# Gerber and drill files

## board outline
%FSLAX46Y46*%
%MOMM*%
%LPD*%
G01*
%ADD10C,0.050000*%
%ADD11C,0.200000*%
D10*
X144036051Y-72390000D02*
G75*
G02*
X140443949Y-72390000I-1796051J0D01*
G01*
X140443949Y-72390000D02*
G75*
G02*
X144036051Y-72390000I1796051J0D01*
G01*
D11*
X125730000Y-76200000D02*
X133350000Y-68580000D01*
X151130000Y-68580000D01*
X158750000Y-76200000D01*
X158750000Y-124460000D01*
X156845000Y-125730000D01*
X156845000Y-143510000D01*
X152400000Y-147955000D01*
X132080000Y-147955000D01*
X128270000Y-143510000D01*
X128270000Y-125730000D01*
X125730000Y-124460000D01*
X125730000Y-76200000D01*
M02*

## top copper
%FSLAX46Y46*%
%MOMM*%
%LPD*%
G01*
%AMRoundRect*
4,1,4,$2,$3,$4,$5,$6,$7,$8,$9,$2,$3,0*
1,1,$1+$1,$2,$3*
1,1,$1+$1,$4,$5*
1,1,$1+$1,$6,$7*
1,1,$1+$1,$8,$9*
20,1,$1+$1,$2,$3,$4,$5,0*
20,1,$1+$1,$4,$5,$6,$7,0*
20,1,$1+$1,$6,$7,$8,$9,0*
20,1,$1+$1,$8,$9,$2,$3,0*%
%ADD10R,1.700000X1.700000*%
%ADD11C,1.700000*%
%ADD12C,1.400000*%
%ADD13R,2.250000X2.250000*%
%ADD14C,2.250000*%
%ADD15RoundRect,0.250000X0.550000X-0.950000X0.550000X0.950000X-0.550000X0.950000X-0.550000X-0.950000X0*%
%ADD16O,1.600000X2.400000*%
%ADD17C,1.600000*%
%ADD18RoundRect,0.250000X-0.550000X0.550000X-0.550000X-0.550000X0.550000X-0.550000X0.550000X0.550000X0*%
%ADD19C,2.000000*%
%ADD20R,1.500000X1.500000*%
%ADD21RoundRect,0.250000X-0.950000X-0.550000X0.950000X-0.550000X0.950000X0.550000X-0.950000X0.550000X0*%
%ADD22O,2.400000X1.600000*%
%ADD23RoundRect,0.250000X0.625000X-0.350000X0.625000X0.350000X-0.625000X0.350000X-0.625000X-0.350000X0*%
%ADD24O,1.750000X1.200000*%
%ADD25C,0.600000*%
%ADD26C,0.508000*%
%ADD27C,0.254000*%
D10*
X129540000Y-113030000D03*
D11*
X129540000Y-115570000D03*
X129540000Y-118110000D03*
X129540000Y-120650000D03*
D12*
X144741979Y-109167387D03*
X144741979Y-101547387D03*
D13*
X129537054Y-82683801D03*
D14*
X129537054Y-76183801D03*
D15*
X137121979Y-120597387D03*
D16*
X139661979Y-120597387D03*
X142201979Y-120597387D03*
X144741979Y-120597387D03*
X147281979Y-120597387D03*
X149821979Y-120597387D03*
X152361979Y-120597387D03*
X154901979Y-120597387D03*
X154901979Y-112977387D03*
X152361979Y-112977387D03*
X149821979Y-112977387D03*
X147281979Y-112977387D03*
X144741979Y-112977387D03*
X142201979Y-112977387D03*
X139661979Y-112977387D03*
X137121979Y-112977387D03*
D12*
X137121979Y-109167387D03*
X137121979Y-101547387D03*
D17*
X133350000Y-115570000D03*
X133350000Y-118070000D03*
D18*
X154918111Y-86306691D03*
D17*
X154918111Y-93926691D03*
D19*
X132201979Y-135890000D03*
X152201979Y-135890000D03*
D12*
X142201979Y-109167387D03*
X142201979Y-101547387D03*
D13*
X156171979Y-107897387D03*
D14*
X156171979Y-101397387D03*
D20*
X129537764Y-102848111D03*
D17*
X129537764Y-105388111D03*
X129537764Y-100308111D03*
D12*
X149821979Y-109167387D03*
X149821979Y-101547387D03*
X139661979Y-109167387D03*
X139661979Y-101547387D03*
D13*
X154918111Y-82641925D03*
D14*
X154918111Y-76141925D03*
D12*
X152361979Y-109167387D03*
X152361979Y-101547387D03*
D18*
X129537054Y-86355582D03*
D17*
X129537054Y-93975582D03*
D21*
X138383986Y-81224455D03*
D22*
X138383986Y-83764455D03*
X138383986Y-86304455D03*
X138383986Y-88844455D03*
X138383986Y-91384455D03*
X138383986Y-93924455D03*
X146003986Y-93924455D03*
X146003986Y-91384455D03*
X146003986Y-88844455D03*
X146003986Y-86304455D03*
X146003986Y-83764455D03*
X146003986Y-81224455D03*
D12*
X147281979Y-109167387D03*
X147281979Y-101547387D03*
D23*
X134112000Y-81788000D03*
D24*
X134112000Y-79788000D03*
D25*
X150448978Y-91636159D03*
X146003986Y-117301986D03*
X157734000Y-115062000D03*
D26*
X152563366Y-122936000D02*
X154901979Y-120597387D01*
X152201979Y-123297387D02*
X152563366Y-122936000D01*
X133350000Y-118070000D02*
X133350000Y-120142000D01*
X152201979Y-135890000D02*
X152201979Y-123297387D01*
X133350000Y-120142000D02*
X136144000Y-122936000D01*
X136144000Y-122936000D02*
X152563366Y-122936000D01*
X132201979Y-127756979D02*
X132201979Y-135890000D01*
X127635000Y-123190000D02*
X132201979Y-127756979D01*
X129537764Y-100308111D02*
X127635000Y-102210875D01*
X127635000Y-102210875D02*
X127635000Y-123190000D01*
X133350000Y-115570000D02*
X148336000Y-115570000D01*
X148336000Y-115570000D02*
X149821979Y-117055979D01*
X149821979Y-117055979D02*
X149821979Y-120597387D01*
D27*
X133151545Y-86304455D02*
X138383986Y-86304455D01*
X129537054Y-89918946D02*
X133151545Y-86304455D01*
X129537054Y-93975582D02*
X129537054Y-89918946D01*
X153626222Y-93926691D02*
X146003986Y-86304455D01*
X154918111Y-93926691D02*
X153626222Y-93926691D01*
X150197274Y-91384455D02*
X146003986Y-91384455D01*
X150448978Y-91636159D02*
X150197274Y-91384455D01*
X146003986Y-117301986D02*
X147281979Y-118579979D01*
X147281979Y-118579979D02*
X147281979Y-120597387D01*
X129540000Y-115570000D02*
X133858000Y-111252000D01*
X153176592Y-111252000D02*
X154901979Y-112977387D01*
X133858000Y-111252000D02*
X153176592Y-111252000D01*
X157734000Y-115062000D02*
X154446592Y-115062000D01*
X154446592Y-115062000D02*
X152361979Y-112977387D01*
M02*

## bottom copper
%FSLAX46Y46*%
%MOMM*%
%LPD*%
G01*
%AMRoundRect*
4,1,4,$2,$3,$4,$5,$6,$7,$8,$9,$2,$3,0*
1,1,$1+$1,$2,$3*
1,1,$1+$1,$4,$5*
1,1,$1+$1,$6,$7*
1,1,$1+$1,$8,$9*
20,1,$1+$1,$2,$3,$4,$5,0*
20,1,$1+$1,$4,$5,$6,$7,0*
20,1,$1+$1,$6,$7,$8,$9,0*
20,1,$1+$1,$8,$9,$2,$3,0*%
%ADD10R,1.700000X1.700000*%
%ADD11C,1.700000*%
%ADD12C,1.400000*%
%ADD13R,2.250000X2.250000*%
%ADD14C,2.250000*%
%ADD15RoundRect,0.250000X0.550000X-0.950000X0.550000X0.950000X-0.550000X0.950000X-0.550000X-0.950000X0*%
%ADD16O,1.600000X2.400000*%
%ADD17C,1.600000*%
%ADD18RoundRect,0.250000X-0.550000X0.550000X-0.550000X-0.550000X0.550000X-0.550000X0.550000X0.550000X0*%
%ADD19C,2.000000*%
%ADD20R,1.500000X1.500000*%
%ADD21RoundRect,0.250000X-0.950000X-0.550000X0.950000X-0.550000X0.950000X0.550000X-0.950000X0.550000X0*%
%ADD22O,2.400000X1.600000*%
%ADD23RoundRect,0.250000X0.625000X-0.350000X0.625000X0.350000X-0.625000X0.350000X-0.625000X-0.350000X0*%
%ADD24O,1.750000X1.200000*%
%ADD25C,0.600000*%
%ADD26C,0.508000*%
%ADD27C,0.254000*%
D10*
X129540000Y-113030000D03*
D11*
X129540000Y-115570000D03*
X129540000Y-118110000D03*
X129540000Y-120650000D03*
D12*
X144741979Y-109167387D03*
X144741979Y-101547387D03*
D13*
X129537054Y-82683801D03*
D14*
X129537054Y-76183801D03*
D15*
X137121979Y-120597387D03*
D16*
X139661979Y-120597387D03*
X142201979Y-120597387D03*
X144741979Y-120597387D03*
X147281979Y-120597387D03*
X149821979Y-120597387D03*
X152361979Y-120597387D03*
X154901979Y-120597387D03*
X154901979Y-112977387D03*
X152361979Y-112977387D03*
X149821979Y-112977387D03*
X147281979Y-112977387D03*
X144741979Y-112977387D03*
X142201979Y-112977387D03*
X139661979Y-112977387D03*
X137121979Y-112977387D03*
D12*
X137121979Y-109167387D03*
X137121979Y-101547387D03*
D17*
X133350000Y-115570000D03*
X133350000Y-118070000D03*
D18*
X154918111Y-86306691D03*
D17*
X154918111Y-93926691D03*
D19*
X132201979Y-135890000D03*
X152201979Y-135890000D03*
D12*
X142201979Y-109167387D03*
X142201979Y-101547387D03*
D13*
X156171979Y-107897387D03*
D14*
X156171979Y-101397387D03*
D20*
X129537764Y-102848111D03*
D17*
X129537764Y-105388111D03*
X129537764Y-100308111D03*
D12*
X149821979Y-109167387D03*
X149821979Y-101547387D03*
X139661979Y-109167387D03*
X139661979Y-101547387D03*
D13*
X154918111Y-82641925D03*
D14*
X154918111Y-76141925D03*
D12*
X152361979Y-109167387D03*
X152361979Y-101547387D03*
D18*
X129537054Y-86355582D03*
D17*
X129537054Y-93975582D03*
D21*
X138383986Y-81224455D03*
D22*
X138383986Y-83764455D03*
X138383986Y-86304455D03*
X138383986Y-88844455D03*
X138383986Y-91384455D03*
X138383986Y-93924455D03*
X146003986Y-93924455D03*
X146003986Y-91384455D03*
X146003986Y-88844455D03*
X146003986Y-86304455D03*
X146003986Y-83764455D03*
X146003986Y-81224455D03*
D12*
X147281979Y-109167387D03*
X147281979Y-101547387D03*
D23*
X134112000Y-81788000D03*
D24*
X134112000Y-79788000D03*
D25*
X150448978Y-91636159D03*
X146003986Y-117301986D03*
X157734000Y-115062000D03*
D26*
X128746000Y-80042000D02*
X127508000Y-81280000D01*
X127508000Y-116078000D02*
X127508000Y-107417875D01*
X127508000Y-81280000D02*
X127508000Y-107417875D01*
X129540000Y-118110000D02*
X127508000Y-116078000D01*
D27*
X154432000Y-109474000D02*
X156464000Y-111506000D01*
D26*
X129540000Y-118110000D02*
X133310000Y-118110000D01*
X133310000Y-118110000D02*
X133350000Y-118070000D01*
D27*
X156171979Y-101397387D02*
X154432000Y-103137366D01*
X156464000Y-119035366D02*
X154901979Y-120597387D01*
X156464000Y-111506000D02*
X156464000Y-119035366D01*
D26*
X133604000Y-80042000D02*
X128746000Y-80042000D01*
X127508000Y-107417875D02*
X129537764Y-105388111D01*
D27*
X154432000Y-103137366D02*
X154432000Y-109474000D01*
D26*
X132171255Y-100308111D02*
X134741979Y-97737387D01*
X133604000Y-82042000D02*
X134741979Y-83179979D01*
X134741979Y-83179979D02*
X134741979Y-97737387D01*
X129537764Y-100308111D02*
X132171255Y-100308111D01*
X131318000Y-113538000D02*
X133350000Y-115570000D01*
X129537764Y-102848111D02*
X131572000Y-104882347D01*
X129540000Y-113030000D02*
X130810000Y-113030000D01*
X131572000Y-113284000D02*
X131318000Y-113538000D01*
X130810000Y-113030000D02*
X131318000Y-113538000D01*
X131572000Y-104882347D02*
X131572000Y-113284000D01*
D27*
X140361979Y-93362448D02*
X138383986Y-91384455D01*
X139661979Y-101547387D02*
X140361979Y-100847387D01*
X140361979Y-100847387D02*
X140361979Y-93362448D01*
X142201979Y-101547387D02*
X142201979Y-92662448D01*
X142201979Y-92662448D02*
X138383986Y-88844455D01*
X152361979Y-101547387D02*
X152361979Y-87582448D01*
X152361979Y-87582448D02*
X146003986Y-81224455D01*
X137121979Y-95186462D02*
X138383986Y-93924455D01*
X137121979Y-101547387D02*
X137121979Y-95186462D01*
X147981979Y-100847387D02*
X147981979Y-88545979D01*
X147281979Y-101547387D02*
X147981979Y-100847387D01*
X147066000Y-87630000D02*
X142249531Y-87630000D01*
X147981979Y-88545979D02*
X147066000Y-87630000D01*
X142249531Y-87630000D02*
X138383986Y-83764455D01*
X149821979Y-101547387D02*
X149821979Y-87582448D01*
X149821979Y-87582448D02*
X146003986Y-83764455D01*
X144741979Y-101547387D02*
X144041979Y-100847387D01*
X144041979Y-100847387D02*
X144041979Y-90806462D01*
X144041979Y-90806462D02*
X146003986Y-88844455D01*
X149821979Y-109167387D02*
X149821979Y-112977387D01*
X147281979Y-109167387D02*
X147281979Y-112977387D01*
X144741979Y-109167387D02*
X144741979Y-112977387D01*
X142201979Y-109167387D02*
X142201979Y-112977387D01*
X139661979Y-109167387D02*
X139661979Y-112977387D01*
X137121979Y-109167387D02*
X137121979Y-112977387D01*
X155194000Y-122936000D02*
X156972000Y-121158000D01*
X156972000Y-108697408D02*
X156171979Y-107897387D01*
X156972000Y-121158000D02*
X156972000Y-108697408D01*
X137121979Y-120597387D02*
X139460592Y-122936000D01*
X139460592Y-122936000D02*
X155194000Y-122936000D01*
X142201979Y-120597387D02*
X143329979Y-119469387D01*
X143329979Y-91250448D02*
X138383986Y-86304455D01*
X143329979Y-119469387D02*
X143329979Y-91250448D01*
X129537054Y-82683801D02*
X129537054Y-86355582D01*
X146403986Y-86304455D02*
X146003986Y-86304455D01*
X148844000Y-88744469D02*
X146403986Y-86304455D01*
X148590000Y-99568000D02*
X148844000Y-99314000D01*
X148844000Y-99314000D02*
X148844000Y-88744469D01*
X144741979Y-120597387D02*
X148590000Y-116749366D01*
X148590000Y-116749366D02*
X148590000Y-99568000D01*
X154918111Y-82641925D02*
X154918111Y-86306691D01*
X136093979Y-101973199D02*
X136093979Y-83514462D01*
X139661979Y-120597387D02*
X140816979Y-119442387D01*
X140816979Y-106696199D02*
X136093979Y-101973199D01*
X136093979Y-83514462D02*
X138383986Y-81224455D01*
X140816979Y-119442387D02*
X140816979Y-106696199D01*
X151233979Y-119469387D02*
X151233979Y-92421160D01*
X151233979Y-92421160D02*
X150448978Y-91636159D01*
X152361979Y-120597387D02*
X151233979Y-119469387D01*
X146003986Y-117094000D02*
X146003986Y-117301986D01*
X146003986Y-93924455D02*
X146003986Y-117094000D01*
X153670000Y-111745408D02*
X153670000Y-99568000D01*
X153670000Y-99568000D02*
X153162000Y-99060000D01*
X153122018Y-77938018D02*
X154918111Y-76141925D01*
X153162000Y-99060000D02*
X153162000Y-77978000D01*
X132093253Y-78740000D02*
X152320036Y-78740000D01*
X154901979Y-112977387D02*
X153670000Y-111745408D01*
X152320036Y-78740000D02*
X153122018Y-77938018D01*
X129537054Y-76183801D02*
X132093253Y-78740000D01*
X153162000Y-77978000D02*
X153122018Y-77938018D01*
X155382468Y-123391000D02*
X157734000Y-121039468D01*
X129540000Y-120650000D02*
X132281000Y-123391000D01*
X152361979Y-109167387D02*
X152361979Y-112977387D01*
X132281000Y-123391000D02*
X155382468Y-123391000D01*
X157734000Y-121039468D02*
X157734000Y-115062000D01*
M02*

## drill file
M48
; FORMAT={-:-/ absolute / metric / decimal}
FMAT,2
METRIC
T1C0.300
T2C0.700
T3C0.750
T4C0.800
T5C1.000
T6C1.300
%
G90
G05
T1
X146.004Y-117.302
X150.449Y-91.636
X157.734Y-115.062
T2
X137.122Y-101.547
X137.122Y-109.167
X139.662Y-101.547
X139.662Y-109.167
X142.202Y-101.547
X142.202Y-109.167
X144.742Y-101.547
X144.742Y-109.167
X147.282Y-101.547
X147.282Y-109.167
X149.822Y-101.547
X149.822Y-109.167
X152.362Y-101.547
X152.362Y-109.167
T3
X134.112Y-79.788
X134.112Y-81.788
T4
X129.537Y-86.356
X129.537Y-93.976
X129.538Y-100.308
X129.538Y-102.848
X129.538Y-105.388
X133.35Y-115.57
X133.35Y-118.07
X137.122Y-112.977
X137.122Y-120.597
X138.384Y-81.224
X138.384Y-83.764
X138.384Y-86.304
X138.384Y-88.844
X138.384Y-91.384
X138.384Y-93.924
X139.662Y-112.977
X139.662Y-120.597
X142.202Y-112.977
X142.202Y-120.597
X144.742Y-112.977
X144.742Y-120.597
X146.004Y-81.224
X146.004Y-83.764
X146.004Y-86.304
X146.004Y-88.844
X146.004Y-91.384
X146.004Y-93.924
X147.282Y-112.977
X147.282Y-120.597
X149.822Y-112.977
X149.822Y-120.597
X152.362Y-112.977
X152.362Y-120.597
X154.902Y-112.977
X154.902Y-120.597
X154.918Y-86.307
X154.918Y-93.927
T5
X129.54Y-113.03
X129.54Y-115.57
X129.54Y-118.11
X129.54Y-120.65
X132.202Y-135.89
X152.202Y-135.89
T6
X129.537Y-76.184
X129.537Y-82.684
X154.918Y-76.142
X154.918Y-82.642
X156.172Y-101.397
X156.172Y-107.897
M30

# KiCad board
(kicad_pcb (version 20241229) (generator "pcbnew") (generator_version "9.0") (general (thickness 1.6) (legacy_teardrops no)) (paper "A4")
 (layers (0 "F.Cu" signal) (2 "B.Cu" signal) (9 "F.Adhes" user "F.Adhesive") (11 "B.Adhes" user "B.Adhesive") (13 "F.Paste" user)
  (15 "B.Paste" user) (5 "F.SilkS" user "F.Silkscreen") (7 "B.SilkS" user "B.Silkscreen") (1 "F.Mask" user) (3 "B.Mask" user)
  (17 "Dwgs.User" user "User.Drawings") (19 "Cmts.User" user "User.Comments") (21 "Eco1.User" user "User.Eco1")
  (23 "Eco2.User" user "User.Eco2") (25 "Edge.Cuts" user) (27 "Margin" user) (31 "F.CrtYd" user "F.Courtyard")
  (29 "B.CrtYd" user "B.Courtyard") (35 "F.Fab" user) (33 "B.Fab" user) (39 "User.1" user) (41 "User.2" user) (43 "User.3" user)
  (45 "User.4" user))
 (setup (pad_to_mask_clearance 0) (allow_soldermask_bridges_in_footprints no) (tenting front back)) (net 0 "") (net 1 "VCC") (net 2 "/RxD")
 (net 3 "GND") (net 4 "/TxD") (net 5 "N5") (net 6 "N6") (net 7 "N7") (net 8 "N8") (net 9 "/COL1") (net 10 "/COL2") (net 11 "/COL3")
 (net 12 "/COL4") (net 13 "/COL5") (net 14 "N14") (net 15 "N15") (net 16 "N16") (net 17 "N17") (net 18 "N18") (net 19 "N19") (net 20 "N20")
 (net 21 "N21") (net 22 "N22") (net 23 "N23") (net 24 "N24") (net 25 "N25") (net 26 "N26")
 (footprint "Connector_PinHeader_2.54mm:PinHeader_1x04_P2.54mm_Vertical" (layer "F.Cu") (at 129.54 113.03)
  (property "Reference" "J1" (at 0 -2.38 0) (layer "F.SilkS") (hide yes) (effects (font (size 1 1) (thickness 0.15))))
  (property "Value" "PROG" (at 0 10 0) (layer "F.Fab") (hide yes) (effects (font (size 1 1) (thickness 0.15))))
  (pad "1" thru_hole rect (at 0 0) (size 1.7 1.7) (drill 1) (layers "*.Cu" "*.Mask") (remove_unused_layers no) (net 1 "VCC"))
  (pad "2" thru_hole circle (at 0 2.54) (size 1.7 1.7) (drill 1) (layers "*.Cu" "*.Mask") (remove_unused_layers no) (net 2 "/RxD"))
  (pad "3" thru_hole circle (at 0 5.08) (size 1.7 1.7) (drill 1) (layers "*.Cu" "*.Mask") (remove_unused_layers no) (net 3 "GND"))
  (pad "4" thru_hole circle (at 0 7.62) (size 1.7 1.7) (drill 1) (layers "*.Cu" "*.Mask") (remove_unused_layers no) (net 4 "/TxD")))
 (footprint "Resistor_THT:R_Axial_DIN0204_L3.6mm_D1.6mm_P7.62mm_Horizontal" (layer "F.Cu") (at 144.741979 109.167387 90)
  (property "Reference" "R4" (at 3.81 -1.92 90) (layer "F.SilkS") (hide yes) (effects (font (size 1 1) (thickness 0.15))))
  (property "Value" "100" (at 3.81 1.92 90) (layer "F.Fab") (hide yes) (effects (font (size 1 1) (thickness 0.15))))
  (pad "1" thru_hole circle (at 0 0 90) (size 1.4 1.4) (drill 0.7) (layers "*.Cu" "*.Mask") (remove_unused_layers no) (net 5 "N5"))
  (pad "2" thru_hole circle (at 7.62 0 90) (size 1.4 1.4) (drill 0.7) (layers "*.Cu" "*.Mask") (remove_unused_layers no) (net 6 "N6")))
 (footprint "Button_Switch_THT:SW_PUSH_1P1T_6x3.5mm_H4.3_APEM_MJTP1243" (layer "F.Cu") (at 129.537054 82.683801 90)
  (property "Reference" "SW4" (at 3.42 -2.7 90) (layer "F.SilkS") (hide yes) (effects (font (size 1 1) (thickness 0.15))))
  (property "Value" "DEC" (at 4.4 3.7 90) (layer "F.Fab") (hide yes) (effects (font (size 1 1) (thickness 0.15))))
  (pad "1" thru_hole rect (at 0 0 180) (size 2.25 2.25) (drill 1.3) (layers "*.Cu" "*.Mask") (remove_unused_layers no) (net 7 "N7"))
  (pad "2" thru_hole circle (at 6.5 0 180) (size 2.25 2.25) (drill 1.3) (layers "*.Cu" "*.Mask") (remove_unused_layers no) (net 2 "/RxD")))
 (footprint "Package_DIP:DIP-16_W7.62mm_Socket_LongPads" (layer "F.Cu") (at 137.121979 120.597387 90)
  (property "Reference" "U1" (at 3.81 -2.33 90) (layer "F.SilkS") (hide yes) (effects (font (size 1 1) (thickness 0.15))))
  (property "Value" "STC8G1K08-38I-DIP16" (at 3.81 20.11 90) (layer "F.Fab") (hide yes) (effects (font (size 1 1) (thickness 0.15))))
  (pad "1" thru_hole roundrect (at 0 0 90) (size 2.4 1.6) (drill 0.8) (layers "*.Cu" "*.Mask") (remove_unused_layers no)
   (roundrect_rratio 0.15625) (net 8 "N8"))
  (pad "2" thru_hole oval (at 0 2.54 90) (size 2.4 1.6) (drill 0.8) (layers "*.Cu" "*.Mask") (remove_unused_layers no) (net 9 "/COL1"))
  (pad "3" thru_hole oval (at 0 5.08 90) (size 2.4 1.6) (drill 0.8) (layers "*.Cu" "*.Mask") (remove_unused_layers no) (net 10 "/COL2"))
  (pad "4" thru_hole oval (at 0 7.62 90) (size 2.4 1.6) (drill 0.8) (layers "*.Cu" "*.Mask") (remove_unused_layers no) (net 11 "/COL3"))
  (pad "5" thru_hole oval (at 0 10.16 90) (size 2.4 1.6) (drill 0.8) (layers "*.Cu" "*.Mask") (remove_unused_layers no) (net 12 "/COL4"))
  (pad "6" thru_hole oval (at 0 12.7 90) (size 2.4 1.6) (drill 0.8) (layers "*.Cu" "*.Mask") (remove_unused_layers no) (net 1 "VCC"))
  (pad "7" thru_hole oval (at 0 15.24 90) (size 2.4 1.6) (drill 0.8) (layers "*.Cu" "*.Mask") (remove_unused_layers no) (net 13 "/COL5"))
  (pad "8" thru_hole oval (at 0 17.78 90) (size 2.4 1.6) (drill 0.8) (layers "*.Cu" "*.Mask") (remove_unused_layers no) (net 3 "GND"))
  (pad "9" thru_hole oval (at 7.62 17.78 90) (size 2.4 1.6) (drill 0.8) (layers "*.Cu" "*.Mask") (remove_unused_layers no) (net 2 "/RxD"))
  (pad "10" thru_hole oval (at 7.62 15.24 90) (size 2.4 1.6) (drill 0.8) (layers "*.Cu" "*.Mask") (remove_unused_layers no) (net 4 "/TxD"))
  (pad "11" thru_hole oval (at 7.62 12.7 90) (size 2.4 1.6) (drill 0.8) (layers "*.Cu" "*.Mask") (remove_unused_layers no) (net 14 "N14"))
  (pad "12" thru_hole oval (at 7.62 10.16 90) (size 2.4 1.6) (drill 0.8) (layers "*.Cu" "*.Mask") (remove_unused_layers no) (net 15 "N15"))
  (pad "13" thru_hole oval (at 7.62 7.62 90) (size 2.4 1.6) (drill 0.8) (layers "*.Cu" "*.Mask") (remove_unused_layers no) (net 5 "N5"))
  (pad "14" thru_hole oval (at 7.62 5.08 90) (size 2.4 1.6) (drill 0.8) (layers "*.Cu" "*.Mask") (remove_unused_layers no) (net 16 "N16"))
  (pad "15" thru_hole oval (at 7.62 2.54 90) (size 2.4 1.6) (drill 0.8) (layers "*.Cu" "*.Mask") (remove_unused_layers no) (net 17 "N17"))
  (pad "16" thru_hole oval (at 7.62 0 90) (size 2.4 1.6) (drill 0.8) (layers "*.Cu" "*.Mask") (remove_unused_layers no) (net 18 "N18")))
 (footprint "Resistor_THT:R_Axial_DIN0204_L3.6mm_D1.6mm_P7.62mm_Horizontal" (layer "F.Cu") (at 137.121979 109.167387 90)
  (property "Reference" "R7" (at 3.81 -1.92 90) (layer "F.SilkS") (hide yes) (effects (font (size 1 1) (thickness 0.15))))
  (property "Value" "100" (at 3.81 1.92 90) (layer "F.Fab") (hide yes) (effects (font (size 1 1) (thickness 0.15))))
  (pad "1" thru_hole circle (at 0 0 90) (size 1.4 1.4) (drill 0.7) (layers "*.Cu" "*.Mask") (remove_unused_layers no) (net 18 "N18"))
  (pad "2" thru_hole circle (at 7.62 0 90) (size 1.4 1.4) (drill 0.7) (layers "*.Cu" "*.Mask") (remove_unused_layers no) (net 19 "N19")))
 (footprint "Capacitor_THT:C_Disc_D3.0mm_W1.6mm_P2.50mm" (layer "F.Cu") (at 133.35 115.57 -90)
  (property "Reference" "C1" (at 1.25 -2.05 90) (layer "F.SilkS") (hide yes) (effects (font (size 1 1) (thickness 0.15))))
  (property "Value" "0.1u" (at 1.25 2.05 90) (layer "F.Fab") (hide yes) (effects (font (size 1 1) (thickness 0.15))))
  (pad "1" thru_hole circle (at 0 0 270) (size 1.6 1.6) (drill 0.8) (layers "*.Cu" "*.Mask") (remove_unused_layers no) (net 1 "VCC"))
  (pad "2" thru_hole circle (at 2.5 0 270) (size 1.6 1.6) (drill 0.8) (layers "*.Cu" "*.Mask") (remove_unused_layers no) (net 3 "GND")))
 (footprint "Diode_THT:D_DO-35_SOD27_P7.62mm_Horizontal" (layer "F.Cu") (at 154.918111 86.306691 -90)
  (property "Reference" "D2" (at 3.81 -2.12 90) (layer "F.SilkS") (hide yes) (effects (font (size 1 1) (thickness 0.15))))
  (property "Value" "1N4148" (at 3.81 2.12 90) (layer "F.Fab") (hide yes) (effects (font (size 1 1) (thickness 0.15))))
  (pad "1" thru_hole roundrect (at 0 0 270) (size 1.6 1.6) (drill 0.8) (layers "*.Cu" "*.Mask") (remove_unused_layers no)
   (roundrect_rratio 0.15625) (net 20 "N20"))
  (pad "2" thru_hole circle (at 7.62 0 270) (size 1.6 1.6) (drill 0.8) (layers "*.Cu" "*.Mask") (remove_unused_layers no) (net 11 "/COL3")))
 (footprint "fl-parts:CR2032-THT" (layer "F.Cu") (at 142.201979 135.89 180)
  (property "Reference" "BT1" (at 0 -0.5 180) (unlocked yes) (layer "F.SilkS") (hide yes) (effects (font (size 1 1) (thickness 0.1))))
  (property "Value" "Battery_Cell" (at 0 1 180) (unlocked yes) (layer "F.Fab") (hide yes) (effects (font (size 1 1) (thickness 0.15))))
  (pad "1" thru_hole circle (at 10 0 180) (size 2 2) (drill 1) (layers "*.Cu" "*.Mask") (remove_unused_layers no) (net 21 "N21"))
  (pad "2" thru_hole circle (at -10 0 180) (size 2 2) (drill 1) (layers "*.Cu" "*.Mask") (remove_unused_layers no) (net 3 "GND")))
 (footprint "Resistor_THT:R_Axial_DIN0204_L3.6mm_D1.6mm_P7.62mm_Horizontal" (layer "F.Cu") (at 142.201979 109.167387 90)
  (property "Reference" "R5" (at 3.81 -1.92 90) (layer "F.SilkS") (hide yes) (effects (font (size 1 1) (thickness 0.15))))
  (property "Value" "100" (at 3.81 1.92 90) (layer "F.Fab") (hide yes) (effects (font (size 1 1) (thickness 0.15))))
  (pad "1" thru_hole circle (at 0 0 90) (size 1.4 1.4) (drill 0.7) (layers "*.Cu" "*.Mask") (remove_unused_layers no) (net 16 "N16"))
  (pad "2" thru_hole circle (at 7.62 0 90) (size 1.4 1.4) (drill 0.7) (layers "*.Cu" "*.Mask") (remove_unused_layers no) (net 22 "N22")))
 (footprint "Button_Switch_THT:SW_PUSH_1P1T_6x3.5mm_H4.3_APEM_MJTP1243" (layer "F.Cu") (at 156.171979 107.897387 90)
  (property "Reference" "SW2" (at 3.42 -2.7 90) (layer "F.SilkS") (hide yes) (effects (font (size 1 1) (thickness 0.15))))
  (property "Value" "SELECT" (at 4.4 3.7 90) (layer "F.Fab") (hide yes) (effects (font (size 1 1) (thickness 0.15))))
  (pad "1" thru_hole rect (at 0 0 180) (size 2.25 2.25) (drill 1.3) (layers "*.Cu" "*.Mask") (remove_unused_layers no) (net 8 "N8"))
  (pad "2" thru_hole circle (at 6.5 0 180) (size 2.25 2.25) (drill 1.3) (layers "*.Cu" "*.Mask") (remove_unused_layers no) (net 3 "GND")))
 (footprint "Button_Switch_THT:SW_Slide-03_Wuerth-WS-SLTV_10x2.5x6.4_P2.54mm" (layer "F.Cu") (at 129.537764 102.848111 90)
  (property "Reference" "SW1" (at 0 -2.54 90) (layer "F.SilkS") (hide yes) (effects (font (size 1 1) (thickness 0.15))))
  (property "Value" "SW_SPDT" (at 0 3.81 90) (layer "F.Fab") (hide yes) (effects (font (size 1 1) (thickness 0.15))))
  (pad "1" thru_hole rect (at 0 0 90) (size 1.5 1.5) (drill 0.8) (layers "*.Cu" "*.Mask") (remove_unused_layers no) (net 1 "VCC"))
  (pad "2" thru_hole circle (at -2.54 0 90) (size 1.6 1.6) (drill 0.8) (layers "*.Cu" "*.Mask") (remove_unused_layers no) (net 3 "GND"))
  (pad "3" thru_hole circle (at 2.54 0 90) (size 1.6 1.6) (drill 0.8) (layers "*.Cu" "*.Mask") (remove_unused_layers no) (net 21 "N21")))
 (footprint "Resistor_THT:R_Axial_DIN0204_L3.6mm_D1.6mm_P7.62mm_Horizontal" (layer "F.Cu") (at 149.821979 109.167387 90)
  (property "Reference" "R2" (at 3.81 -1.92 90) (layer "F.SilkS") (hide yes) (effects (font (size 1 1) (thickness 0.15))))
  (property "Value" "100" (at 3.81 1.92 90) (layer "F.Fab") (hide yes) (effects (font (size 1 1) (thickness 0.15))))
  (pad "1" thru_hole circle (at 0 0 90) (size 1.4 1.4) (drill 0.7) (layers "*.Cu" "*.Mask") (remove_unused_layers no) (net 14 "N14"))
  (pad "2" thru_hole circle (at 7.62 0 90) (size 1.4 1.4) (drill 0.7) (layers "*.Cu" "*.Mask") (remove_unused_layers no) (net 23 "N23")))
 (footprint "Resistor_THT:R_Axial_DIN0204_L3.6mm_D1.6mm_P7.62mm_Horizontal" (layer "F.Cu") (at 139.661979 109.167387 90)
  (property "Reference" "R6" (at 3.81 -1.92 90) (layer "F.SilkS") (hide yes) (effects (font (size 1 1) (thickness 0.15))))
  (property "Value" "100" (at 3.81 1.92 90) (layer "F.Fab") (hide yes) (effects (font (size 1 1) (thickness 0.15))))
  (pad "1" thru_hole circle (at 0 0 90) (size 1.4 1.4) (drill 0.7) (layers "*.Cu" "*.Mask") (remove_unused_layers no) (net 17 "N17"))
  (pad "2" thru_hole circle (at 7.62 0 90) (size 1.4 1.4) (drill 0.7) (layers "*.Cu" "*.Mask") (remove_unused_layers no) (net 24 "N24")))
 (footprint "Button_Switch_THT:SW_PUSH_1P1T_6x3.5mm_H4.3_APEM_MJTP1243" (layer "F.Cu") (at 154.918111 82.641925 90)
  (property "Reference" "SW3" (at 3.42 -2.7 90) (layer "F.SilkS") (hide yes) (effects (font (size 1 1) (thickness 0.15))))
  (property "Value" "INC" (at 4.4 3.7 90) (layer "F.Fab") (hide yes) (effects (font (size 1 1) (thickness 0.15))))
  (pad "1" thru_hole rect (at 0 0 180) (size 2.25 2.25) (drill 1.3) (layers "*.Cu" "*.Mask") (remove_unused_layers no) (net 20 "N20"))
  (pad "2" thru_hole circle (at 6.5 0 180) (size 2.25 2.25) (drill 1.3) (layers "*.Cu" "*.Mask") (remove_unused_layers no) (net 2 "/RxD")))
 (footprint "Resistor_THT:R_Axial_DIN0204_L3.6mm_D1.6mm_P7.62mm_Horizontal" (layer "F.Cu") (at 152.361979 109.167387 90)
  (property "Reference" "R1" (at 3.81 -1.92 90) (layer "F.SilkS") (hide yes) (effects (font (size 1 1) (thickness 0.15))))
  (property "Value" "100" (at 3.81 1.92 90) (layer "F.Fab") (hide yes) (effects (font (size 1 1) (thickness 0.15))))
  (pad "1" thru_hole circle (at 0 0 90) (size 1.4 1.4) (drill 0.7) (layers "*.Cu" "*.Mask") (remove_unused_layers no) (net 4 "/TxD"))
  (pad "2" thru_hole circle (at 7.62 0 90) (size 1.4 1.4) (drill 0.7) (layers "*.Cu" "*.Mask") (remove_unused_layers no) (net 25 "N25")))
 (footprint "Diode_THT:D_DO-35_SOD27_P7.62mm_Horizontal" (layer "F.Cu") (at 129.537054 86.355582 -90)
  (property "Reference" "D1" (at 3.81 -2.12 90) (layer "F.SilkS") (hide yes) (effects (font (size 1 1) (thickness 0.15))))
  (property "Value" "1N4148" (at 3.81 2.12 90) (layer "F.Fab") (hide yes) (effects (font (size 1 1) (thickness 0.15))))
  (pad "1" thru_hole roundrect (at 0 0 270) (size 1.6 1.6) (drill 0.8) (layers "*.Cu" "*.Mask") (remove_unused_layers no)
   (roundrect_rratio 0.15625) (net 7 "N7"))
  (pad "2" thru_hole circle (at 7.62 0 270) (size 1.6 1.6) (drill 0.8) (layers "*.Cu" "*.Mask") (remove_unused_layers no) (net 10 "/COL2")))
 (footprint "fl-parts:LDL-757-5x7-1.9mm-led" (layer "F.Cu") (at 138.383986 81.224455)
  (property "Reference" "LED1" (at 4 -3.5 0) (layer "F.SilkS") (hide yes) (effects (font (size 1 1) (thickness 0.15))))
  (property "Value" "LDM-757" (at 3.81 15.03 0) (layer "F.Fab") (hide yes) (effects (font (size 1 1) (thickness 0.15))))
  (pad "1" thru_hole roundrect (at 0 0) (size 2.4 1.6) (drill 0.8) (layers "*.Cu" "*.Mask") (remove_unused_layers no)
   (roundrect_rratio 0.15625) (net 9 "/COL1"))
  (pad "2" thru_hole oval (at 0 2.54) (size 2.4 1.6) (drill 0.8) (layers "*.Cu" "*.Mask") (remove_unused_layers no) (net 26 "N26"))
  (pad "3" thru_hole oval (at 0 5.08) (size 2.4 1.6) (drill 0.8) (layers "*.Cu" "*.Mask") (remove_unused_layers no) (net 10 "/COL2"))
  (pad "4" thru_hole oval (at 0 7.62) (size 2.4 1.6) (drill 0.8) (layers "*.Cu" "*.Mask") (remove_unused_layers no) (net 22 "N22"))
  (pad "5" thru_hole oval (at 0 10.16) (size 2.4 1.6) (drill 0.8) (layers "*.Cu" "*.Mask") (remove_unused_layers no) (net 24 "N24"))
  (pad "6" thru_hole oval (at 0 12.7) (size 2.4 1.6) (drill 0.8) (layers "*.Cu" "*.Mask") (remove_unused_layers no) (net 19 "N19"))
  (pad "7" thru_hole oval (at 7.62 12.7) (size 2.4 1.6) (drill 0.8) (layers "*.Cu" "*.Mask") (remove_unused_layers no) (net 12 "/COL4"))
  (pad "8" thru_hole oval (at 7.62 10.16) (size 2.4 1.6) (drill 0.8) (layers "*.Cu" "*.Mask") (remove_unused_layers no) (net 13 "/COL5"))
  (pad "9" thru_hole oval (at 7.62 7.62) (size 2.4 1.6) (drill 0.8) (layers "*.Cu" "*.Mask") (remove_unused_layers no) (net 6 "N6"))
  (pad "10" thru_hole oval (at 7.62 5.08) (size 2.4 1.6) (drill 0.8) (layers "*.Cu" "*.Mask") (remove_unused_layers no) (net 11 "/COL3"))
  (pad "11" thru_hole oval (at 7.62 2.54) (size 2.4 1.6) (drill 0.8) (layers "*.Cu" "*.Mask") (remove_unused_layers no) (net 23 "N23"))
  (pad "12" thru_hole oval (at 7.62 0) (size 2.4 1.6) (drill 0.8) (layers "*.Cu" "*.Mask") (remove_unused_layers no) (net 25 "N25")))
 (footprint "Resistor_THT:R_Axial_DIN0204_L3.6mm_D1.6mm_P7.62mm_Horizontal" (layer "F.Cu") (at 147.281979 109.167387 90)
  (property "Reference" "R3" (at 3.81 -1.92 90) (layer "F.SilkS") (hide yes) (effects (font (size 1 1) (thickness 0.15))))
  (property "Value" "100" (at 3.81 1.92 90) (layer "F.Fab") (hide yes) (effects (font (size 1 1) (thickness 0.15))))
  (pad "1" thru_hole circle (at 0 0 90) (size 1.4 1.4) (drill 0.7) (layers "*.Cu" "*.Mask") (remove_unused_layers no) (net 15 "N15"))
  (pad "2" thru_hole circle (at 7.62 0 90) (size 1.4 1.4) (drill 0.7) (layers "*.Cu" "*.Mask") (remove_unused_layers no) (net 26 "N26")))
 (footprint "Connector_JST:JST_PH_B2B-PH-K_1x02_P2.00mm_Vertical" (layer "B.Cu") (at 134.112 81.788 90)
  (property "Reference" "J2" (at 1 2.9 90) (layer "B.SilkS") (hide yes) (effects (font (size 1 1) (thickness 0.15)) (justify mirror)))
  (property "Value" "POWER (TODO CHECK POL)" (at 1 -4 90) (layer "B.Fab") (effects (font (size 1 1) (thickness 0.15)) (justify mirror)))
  (pad "1" thru_hole roundrect (at 0 0 90) (size 1.2 1.75) (drill 0.75) (layers "*.Cu" "*.Mask") (remove_unused_layers no)
   (roundrect_rratio 0.208333) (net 21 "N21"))
  (pad "2" thru_hole oval (at 2 0 90) (size 1.2 1.75) (drill 0.75) (layers "*.Cu" "*.Mask") (remove_unused_layers no) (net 3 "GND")))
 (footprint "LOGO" (layer "B.Cu") (at 145.415 90.805 180)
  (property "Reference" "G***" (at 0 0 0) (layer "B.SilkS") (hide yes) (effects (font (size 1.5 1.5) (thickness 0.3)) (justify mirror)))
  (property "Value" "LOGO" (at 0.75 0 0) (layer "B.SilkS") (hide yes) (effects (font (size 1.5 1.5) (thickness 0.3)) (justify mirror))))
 (gr_circle (center 142.24 72.39) (end 143.51 73.66) (stroke (width 0.05) (type default)) (fill no) (layer "Edge.Cuts"))
 (gr_poly
  (pts (xy 125.73 76.2) (xy 133.35 68.58) (xy 151.13 68.58) (xy 158.75 76.2) (xy 158.75 124.46) (xy 156.845 125.73) (xy 156.845 143.51)
   (xy 152.4 147.955) (xy 132.08 147.955) (xy 128.27 143.51) (xy 128.27 125.73) (xy 125.73 124.46))
  (stroke (width 0.2) (type solid)) (fill no) (layer "Edge.Cuts"))
 (segment (start 152.563366 122.936) (end 154.901979 120.597387) (width 0.508) (layer "F.Cu") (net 3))
 (segment (start 152.201979 123.297387) (end 152.563366 122.936) (width 0.508) (layer "F.Cu") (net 3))
 (segment (start 133.35 118.07) (end 133.35 120.142) (width 0.508) (layer "F.Cu") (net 3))
 (segment (start 152.201979 135.89) (end 152.201979 123.297387) (width 0.508) (layer "F.Cu") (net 3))
 (segment (start 133.35 120.142) (end 136.144 122.936) (width 0.508) (layer "F.Cu") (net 3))
 (segment (start 136.144 122.936) (end 152.563366 122.936) (width 0.508) (layer "F.Cu") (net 3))
 (segment (start 128.746 80.042) (end 127.508 81.28) (width 0.508) (layer "B.Cu") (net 3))
 (segment (start 127.508 116.078) (end 127.508 107.417875) (width 0.508) (layer "B.Cu") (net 3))
 (segment (start 127.508 81.28) (end 127.508 107.417875) (width 0.508) (layer "B.Cu") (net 3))
 (segment (start 129.54 118.11) (end 127.508 116.078) (width 0.508) (layer "B.Cu") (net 3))
 (segment (start 154.432 109.474) (end 156.464 111.506) (width 0.254) (layer "B.Cu") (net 3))
 (segment (start 129.54 118.11) (end 133.31 118.11) (width 0.508) (layer "B.Cu") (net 3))
 (segment (start 133.31 118.11) (end 133.35 118.07) (width 0.508) (layer "B.Cu") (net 3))
 (segment (start 156.171979 101.397387) (end 154.432 103.137366) (width 0.254) (layer "B.Cu") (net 3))
 (segment (start 156.464 119.035366) (end 154.901979 120.597387) (width 0.254) (layer "B.Cu") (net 3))
 (segment (start 156.464 111.506) (end 156.464 119.035366) (width 0.254) (layer "B.Cu") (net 3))
 (segment (start 133.604 80.042) (end 128.746 80.042) (width 0.508) (layer "B.Cu") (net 3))
 (segment (start 127.508 107.417875) (end 129.537764 105.388111) (width 0.508) (layer "B.Cu") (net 3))
 (segment (start 154.432 103.137366) (end 154.432 109.474) (width 0.254) (layer "B.Cu") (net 3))
 (segment (start 132.201979 127.756979) (end 132.201979 135.89) (width 0.508) (layer "F.Cu") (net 21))
 (segment (start 127.635 123.19) (end 132.201979 127.756979) (width 0.508) (layer "F.Cu") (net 21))
 (segment (start 129.537764 100.308111) (end 127.635 102.210875) (width 0.508) (layer "F.Cu") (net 21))
 (segment (start 127.635 102.210875) (end 127.635 123.19) (width 0.508) (layer "F.Cu") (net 21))
 (segment (start 132.171255 100.308111) (end 134.741979 97.737387) (width 0.508) (layer "B.Cu") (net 21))
 (segment (start 133.604 82.042) (end 134.741979 83.179979) (width 0.508) (layer "B.Cu") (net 21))
 (segment (start 134.741979 83.179979) (end 134.741979 97.737387) (width 0.508) (layer "B.Cu") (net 21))
 (segment (start 129.537764 100.308111) (end 132.171255 100.308111) (width 0.508) (layer "B.Cu") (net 21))
 (segment (start 133.35 115.57) (end 148.336 115.57) (width 0.508) (layer "F.Cu") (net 1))
 (segment (start 148.336 115.57) (end 149.821979 117.055979) (width 0.508) (layer "F.Cu") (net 1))
 (segment (start 149.821979 117.055979) (end 149.821979 120.597387) (width 0.508) (layer "F.Cu") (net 1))
 (segment (start 131.318 113.538) (end 133.35 115.57) (width 0.508) (layer "B.Cu") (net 1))
 (segment (start 129.537764 102.848111) (end 131.572 104.882347) (width 0.508) (layer "B.Cu") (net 1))
 (segment (start 129.54 113.03) (end 130.81 113.03) (width 0.508) (layer "B.Cu") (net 1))
 (segment (start 131.572 113.284) (end 131.318 113.538) (width 0.508) (layer "B.Cu") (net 1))
 (segment (start 130.81 113.03) (end 131.318 113.538) (width 0.508) (layer "B.Cu") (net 1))
 (segment (start 131.572 104.882347) (end 131.572 113.284) (width 0.508) (layer "B.Cu") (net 1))
 (segment (start 140.361979 93.362448) (end 138.383986 91.384455) (width 0.254) (layer "B.Cu") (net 24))
 (segment (start 139.661979 101.547387) (end 140.361979 100.847387) (width 0.254) (layer "B.Cu") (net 24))
 (segment (start 140.361979 100.847387) (end 140.361979 93.362448) (width 0.254) (layer "B.Cu") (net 24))
 (segment (start 142.201979 101.547387) (end 142.201979 92.662448) (width 0.254) (layer "B.Cu") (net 22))
 (segment (start 142.201979 92.662448) (end 138.383986 88.844455) (width 0.254) (layer "B.Cu") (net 22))
 (segment (start 152.361979 101.547387) (end 152.361979 87.582448) (width 0.254) (layer "B.Cu") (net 25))
 (segment (start 152.361979 87.582448) (end 146.003986 81.224455) (width 0.254) (layer "B.Cu") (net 25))
 (segment (start 137.121979 95.186462) (end 138.383986 93.924455) (width 0.254) (layer "B.Cu") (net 19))
 (segment (start 137.121979 101.547387) (end 137.121979 95.186462) (width 0.254) (layer "B.Cu") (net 19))
 (segment (start 147.981979 100.847387) (end 147.981979 88.545979) (width 0.254) (layer "B.Cu") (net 26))
 (segment (start 147.281979 101.547387) (end 147.981979 100.847387) (width 0.254) (layer "B.Cu") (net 26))
 (segment (start 147.066 87.63) (end 142.249531 87.63) (width 0.254) (layer "B.Cu") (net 26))
 (segment (start 147.981979 88.545979) (end 147.066 87.63) (width 0.254) (layer "B.Cu") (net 26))
 (segment (start 142.249531 87.63) (end 138.383986 83.764455) (width 0.254) (layer "B.Cu") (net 26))
 (segment (start 149.821979 101.547387) (end 149.821979 87.582448) (width 0.254) (layer "B.Cu") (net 23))
 (segment (start 149.821979 87.582448) (end 146.003986 83.764455) (width 0.254) (layer "B.Cu") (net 23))
 (segment (start 144.741979 101.547387) (end 144.041979 100.847387) (width 0.254) (layer "B.Cu") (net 6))
 (segment (start 144.041979 100.847387) (end 144.041979 90.806462) (width 0.254) (layer "B.Cu") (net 6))
 (segment (start 144.041979 90.806462) (end 146.003986 88.844455) (width 0.254) (layer "B.Cu") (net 6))
 (segment (start 149.821979 109.167387) (end 149.821979 112.977387) (width 0.254) (layer "B.Cu") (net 14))
 (segment (start 147.281979 109.167387) (end 147.281979 112.977387) (width 0.254) (layer "B.Cu") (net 15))
 (segment (start 144.741979 109.167387) (end 144.741979 112.977387) (width 0.254) (layer "B.Cu") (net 5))
 (segment (start 142.201979 109.167387) (end 142.201979 112.977387) (width 0.254) (layer "B.Cu") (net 16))
 (segment (start 139.661979 109.167387) (end 139.661979 112.977387) (width 0.254) (layer "B.Cu") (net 17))
 (segment (start 137.121979 109.167387) (end 137.121979 112.977387) (width 0.254) (layer "B.Cu") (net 18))
 (segment (start 155.194 122.936) (end 156.972 121.158) (width 0.254) (layer "B.Cu") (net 8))
 (segment (start 156.972 108.697408) (end 156.171979 107.897387) (width 0.254) (layer "B.Cu") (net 8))
 (segment (start 156.972 121.158) (end 156.972 108.697408) (width 0.254) (layer "B.Cu") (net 8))
 (segment (start 137.121979 120.597387) (end 139.460592 122.936) (width 0.254) (layer "B.Cu") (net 8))
 (segment (start 139.460592 122.936) (end 155.194 122.936) (width 0.254) (layer "B.Cu") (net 8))
 (segment (start 133.151545 86.304455) (end 138.383986 86.304455) (width 0.254) (layer "F.Cu") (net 10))
 (segment (start 129.537054 89.918946) (end 133.151545 86.304455) (width 0.254) (layer "F.Cu") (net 10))
 (segment (start 129.537054 93.975582) (end 129.537054 89.918946) (width 0.254) (layer "F.Cu") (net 10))
 (segment (start 142.201979 120.597387) (end 143.329979 119.469387) (width 0.254) (layer "B.Cu") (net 10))
 (segment (start 143.329979 91.250448) (end 138.383986 86.304455) (width 0.254) (layer "B.Cu") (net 10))
 (segment (start 143.329979 119.469387) (end 143.329979 91.250448) (width 0.254) (layer "B.Cu") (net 10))
 (segment (start 129.537054 82.683801) (end 129.537054 86.355582) (width 0.254) (layer "B.Cu") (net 7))
 (segment (start 153.626222 93.926691) (end 146.003986 86.304455) (width 0.254) (layer "F.Cu") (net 11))
 (segment (start 154.918111 93.926691) (end 153.626222 93.926691) (width 0.254) (layer "F.Cu") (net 11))
 (segment (start 146.403986 86.304455) (end 146.003986 86.304455) (width 0.254) (layer "B.Cu") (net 11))
 (segment (start 148.844 88.744469) (end 146.403986 86.304455) (width 0.254) (layer "B.Cu") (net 11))
 (segment (start 148.59 99.568) (end 148.844 99.314) (width 0.254) (layer "B.Cu") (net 11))
 (segment (start 148.844 99.314) (end 148.844 88.744469) (width 0.254) (layer "B.Cu") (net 11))
 (segment (start 144.741979 120.597387) (end 148.59 116.749366) (width 0.254) (layer "B.Cu") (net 11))
 (segment (start 148.59 116.749366) (end 148.59 99.568) (width 0.254) (layer "B.Cu") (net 11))
 (segment (start 154.918111 82.641925) (end 154.918111 86.306691) (width 0.254) (layer "B.Cu") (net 20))
 (segment (start 136.093979 101.973199) (end 136.093979 83.514462) (width 0.254) (layer "B.Cu") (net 9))
 (segment (start 139.661979 120.597387) (end 140.816979 119.442387) (width 0.254) (layer "B.Cu") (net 9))
 (segment (start 140.816979 106.696199) (end 136.093979 101.973199) (width 0.254) (layer "B.Cu") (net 9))
 (segment (start 136.093979 83.514462) (end 138.383986 81.224455) (width 0.254) (layer "B.Cu") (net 9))
 (segment (start 140.816979 119.442387) (end 140.816979 106.696199) (width 0.254) (layer "B.Cu") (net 9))
 (segment (start 150.197274 91.384455) (end 146.003986 91.384455) (width 0.254) (layer "F.Cu") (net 13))
 (segment (start 150.448978 91.636159) (end 150.197274 91.384455) (width 0.254) (layer "F.Cu") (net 13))
 (via (at 150.448978 91.636159) (size 0.6) (drill 0.3) (layers "F.Cu" "B.Cu") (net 13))
 (segment (start 151.233979 119.469387) (end 151.233979 92.42116) (width 0.254) (layer "B.Cu") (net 13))
 (segment (start 151.233979 92.42116) (end 150.448978 91.636159) (width 0.254) (layer "B.Cu") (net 13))
 (segment (start 152.361979 120.597387) (end 151.233979 119.469387) (width 0.254) (layer "B.Cu") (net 13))
 (segment (start 146.003986 117.301986) (end 147.281979 118.579979) (width 0.254) (layer "F.Cu") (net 12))
 (segment (start 147.281979 118.579979) (end 147.281979 120.597387) (width 0.254) (layer "F.Cu") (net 12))
 (via (at 146.003986 117.301986) (size 0.6) (drill 0.3) (layers "F.Cu" "B.Cu") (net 12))
 (segment (start 146.003986 117.094) (end 146.003986 117.301986) (width 0.254) (layer "B.Cu") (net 12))
 (segment (start 146.003986 93.924455) (end 146.003986 117.094) (width 0.254) (layer "B.Cu") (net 12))
 (segment (start 129.54 115.57) (end 133.858 111.252) (width 0.254) (layer "F.Cu") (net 2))
 (segment (start 153.176592 111.252) (end 154.901979 112.977387) (width 0.254) (layer "F.Cu") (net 2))
 (segment (start 133.858 111.252) (end 153.176592 111.252) (width 0.254) (layer "F.Cu") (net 2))
 (segment (start 153.67 111.745408) (end 153.67 99.568) (width 0.254) (layer "B.Cu") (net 2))
 (segment (start 153.67 99.568) (end 153.162 99.06) (width 0.254) (layer "B.Cu") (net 2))
 (segment (start 153.122018 77.938018) (end 154.918111 76.141925) (width 0.254) (layer "B.Cu") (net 2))
 (segment (start 153.162 99.06) (end 153.162 77.978) (width 0.254) (layer "B.Cu") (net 2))
 (segment (start 132.093253 78.74) (end 152.320036 78.74) (width 0.254) (layer "B.Cu") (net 2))
 (segment (start 154.901979 112.977387) (end 153.67 111.745408) (width 0.254) (layer "B.Cu") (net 2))
 (segment (start 152.320036 78.74) (end 153.122018 77.938018) (width 0.254) (layer "B.Cu") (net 2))
 (segment (start 129.537054 76.183801) (end 132.093253 78.74) (width 0.254) (layer "B.Cu") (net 2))
 (segment (start 153.162 77.978) (end 153.122018 77.938018) (width 0.254) (layer "B.Cu") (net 2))
 (segment (start 157.734 115.062) (end 154.446592 115.062) (width 0.254) (layer "F.Cu") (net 4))
 (segment (start 154.446592 115.062) (end 152.361979 112.977387) (width 0.254) (layer "F.Cu") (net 4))
 (via (at 157.734 115.062) (size 0.6) (drill 0.3) (layers "F.Cu" "B.Cu") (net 4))
 (segment (start 155.382468 123.391) (end 157.734 121.039468) (width 0.254) (layer "B.Cu") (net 4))
 (segment (start 129.54 120.65) (end 132.281 123.391) (width 0.254) (layer "B.Cu") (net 4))
 (segment (start 152.361979 109.167387) (end 152.361979 112.977387) (width 0.254) (layer "B.Cu") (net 4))
 (segment (start 132.281 123.391) (end 155.382468 123.391) (width 0.254) (layer "B.Cu") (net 4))
 (segment (start 157.734 121.039468) (end 157.734 115.062) (width 0.254) (layer "B.Cu") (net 4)))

